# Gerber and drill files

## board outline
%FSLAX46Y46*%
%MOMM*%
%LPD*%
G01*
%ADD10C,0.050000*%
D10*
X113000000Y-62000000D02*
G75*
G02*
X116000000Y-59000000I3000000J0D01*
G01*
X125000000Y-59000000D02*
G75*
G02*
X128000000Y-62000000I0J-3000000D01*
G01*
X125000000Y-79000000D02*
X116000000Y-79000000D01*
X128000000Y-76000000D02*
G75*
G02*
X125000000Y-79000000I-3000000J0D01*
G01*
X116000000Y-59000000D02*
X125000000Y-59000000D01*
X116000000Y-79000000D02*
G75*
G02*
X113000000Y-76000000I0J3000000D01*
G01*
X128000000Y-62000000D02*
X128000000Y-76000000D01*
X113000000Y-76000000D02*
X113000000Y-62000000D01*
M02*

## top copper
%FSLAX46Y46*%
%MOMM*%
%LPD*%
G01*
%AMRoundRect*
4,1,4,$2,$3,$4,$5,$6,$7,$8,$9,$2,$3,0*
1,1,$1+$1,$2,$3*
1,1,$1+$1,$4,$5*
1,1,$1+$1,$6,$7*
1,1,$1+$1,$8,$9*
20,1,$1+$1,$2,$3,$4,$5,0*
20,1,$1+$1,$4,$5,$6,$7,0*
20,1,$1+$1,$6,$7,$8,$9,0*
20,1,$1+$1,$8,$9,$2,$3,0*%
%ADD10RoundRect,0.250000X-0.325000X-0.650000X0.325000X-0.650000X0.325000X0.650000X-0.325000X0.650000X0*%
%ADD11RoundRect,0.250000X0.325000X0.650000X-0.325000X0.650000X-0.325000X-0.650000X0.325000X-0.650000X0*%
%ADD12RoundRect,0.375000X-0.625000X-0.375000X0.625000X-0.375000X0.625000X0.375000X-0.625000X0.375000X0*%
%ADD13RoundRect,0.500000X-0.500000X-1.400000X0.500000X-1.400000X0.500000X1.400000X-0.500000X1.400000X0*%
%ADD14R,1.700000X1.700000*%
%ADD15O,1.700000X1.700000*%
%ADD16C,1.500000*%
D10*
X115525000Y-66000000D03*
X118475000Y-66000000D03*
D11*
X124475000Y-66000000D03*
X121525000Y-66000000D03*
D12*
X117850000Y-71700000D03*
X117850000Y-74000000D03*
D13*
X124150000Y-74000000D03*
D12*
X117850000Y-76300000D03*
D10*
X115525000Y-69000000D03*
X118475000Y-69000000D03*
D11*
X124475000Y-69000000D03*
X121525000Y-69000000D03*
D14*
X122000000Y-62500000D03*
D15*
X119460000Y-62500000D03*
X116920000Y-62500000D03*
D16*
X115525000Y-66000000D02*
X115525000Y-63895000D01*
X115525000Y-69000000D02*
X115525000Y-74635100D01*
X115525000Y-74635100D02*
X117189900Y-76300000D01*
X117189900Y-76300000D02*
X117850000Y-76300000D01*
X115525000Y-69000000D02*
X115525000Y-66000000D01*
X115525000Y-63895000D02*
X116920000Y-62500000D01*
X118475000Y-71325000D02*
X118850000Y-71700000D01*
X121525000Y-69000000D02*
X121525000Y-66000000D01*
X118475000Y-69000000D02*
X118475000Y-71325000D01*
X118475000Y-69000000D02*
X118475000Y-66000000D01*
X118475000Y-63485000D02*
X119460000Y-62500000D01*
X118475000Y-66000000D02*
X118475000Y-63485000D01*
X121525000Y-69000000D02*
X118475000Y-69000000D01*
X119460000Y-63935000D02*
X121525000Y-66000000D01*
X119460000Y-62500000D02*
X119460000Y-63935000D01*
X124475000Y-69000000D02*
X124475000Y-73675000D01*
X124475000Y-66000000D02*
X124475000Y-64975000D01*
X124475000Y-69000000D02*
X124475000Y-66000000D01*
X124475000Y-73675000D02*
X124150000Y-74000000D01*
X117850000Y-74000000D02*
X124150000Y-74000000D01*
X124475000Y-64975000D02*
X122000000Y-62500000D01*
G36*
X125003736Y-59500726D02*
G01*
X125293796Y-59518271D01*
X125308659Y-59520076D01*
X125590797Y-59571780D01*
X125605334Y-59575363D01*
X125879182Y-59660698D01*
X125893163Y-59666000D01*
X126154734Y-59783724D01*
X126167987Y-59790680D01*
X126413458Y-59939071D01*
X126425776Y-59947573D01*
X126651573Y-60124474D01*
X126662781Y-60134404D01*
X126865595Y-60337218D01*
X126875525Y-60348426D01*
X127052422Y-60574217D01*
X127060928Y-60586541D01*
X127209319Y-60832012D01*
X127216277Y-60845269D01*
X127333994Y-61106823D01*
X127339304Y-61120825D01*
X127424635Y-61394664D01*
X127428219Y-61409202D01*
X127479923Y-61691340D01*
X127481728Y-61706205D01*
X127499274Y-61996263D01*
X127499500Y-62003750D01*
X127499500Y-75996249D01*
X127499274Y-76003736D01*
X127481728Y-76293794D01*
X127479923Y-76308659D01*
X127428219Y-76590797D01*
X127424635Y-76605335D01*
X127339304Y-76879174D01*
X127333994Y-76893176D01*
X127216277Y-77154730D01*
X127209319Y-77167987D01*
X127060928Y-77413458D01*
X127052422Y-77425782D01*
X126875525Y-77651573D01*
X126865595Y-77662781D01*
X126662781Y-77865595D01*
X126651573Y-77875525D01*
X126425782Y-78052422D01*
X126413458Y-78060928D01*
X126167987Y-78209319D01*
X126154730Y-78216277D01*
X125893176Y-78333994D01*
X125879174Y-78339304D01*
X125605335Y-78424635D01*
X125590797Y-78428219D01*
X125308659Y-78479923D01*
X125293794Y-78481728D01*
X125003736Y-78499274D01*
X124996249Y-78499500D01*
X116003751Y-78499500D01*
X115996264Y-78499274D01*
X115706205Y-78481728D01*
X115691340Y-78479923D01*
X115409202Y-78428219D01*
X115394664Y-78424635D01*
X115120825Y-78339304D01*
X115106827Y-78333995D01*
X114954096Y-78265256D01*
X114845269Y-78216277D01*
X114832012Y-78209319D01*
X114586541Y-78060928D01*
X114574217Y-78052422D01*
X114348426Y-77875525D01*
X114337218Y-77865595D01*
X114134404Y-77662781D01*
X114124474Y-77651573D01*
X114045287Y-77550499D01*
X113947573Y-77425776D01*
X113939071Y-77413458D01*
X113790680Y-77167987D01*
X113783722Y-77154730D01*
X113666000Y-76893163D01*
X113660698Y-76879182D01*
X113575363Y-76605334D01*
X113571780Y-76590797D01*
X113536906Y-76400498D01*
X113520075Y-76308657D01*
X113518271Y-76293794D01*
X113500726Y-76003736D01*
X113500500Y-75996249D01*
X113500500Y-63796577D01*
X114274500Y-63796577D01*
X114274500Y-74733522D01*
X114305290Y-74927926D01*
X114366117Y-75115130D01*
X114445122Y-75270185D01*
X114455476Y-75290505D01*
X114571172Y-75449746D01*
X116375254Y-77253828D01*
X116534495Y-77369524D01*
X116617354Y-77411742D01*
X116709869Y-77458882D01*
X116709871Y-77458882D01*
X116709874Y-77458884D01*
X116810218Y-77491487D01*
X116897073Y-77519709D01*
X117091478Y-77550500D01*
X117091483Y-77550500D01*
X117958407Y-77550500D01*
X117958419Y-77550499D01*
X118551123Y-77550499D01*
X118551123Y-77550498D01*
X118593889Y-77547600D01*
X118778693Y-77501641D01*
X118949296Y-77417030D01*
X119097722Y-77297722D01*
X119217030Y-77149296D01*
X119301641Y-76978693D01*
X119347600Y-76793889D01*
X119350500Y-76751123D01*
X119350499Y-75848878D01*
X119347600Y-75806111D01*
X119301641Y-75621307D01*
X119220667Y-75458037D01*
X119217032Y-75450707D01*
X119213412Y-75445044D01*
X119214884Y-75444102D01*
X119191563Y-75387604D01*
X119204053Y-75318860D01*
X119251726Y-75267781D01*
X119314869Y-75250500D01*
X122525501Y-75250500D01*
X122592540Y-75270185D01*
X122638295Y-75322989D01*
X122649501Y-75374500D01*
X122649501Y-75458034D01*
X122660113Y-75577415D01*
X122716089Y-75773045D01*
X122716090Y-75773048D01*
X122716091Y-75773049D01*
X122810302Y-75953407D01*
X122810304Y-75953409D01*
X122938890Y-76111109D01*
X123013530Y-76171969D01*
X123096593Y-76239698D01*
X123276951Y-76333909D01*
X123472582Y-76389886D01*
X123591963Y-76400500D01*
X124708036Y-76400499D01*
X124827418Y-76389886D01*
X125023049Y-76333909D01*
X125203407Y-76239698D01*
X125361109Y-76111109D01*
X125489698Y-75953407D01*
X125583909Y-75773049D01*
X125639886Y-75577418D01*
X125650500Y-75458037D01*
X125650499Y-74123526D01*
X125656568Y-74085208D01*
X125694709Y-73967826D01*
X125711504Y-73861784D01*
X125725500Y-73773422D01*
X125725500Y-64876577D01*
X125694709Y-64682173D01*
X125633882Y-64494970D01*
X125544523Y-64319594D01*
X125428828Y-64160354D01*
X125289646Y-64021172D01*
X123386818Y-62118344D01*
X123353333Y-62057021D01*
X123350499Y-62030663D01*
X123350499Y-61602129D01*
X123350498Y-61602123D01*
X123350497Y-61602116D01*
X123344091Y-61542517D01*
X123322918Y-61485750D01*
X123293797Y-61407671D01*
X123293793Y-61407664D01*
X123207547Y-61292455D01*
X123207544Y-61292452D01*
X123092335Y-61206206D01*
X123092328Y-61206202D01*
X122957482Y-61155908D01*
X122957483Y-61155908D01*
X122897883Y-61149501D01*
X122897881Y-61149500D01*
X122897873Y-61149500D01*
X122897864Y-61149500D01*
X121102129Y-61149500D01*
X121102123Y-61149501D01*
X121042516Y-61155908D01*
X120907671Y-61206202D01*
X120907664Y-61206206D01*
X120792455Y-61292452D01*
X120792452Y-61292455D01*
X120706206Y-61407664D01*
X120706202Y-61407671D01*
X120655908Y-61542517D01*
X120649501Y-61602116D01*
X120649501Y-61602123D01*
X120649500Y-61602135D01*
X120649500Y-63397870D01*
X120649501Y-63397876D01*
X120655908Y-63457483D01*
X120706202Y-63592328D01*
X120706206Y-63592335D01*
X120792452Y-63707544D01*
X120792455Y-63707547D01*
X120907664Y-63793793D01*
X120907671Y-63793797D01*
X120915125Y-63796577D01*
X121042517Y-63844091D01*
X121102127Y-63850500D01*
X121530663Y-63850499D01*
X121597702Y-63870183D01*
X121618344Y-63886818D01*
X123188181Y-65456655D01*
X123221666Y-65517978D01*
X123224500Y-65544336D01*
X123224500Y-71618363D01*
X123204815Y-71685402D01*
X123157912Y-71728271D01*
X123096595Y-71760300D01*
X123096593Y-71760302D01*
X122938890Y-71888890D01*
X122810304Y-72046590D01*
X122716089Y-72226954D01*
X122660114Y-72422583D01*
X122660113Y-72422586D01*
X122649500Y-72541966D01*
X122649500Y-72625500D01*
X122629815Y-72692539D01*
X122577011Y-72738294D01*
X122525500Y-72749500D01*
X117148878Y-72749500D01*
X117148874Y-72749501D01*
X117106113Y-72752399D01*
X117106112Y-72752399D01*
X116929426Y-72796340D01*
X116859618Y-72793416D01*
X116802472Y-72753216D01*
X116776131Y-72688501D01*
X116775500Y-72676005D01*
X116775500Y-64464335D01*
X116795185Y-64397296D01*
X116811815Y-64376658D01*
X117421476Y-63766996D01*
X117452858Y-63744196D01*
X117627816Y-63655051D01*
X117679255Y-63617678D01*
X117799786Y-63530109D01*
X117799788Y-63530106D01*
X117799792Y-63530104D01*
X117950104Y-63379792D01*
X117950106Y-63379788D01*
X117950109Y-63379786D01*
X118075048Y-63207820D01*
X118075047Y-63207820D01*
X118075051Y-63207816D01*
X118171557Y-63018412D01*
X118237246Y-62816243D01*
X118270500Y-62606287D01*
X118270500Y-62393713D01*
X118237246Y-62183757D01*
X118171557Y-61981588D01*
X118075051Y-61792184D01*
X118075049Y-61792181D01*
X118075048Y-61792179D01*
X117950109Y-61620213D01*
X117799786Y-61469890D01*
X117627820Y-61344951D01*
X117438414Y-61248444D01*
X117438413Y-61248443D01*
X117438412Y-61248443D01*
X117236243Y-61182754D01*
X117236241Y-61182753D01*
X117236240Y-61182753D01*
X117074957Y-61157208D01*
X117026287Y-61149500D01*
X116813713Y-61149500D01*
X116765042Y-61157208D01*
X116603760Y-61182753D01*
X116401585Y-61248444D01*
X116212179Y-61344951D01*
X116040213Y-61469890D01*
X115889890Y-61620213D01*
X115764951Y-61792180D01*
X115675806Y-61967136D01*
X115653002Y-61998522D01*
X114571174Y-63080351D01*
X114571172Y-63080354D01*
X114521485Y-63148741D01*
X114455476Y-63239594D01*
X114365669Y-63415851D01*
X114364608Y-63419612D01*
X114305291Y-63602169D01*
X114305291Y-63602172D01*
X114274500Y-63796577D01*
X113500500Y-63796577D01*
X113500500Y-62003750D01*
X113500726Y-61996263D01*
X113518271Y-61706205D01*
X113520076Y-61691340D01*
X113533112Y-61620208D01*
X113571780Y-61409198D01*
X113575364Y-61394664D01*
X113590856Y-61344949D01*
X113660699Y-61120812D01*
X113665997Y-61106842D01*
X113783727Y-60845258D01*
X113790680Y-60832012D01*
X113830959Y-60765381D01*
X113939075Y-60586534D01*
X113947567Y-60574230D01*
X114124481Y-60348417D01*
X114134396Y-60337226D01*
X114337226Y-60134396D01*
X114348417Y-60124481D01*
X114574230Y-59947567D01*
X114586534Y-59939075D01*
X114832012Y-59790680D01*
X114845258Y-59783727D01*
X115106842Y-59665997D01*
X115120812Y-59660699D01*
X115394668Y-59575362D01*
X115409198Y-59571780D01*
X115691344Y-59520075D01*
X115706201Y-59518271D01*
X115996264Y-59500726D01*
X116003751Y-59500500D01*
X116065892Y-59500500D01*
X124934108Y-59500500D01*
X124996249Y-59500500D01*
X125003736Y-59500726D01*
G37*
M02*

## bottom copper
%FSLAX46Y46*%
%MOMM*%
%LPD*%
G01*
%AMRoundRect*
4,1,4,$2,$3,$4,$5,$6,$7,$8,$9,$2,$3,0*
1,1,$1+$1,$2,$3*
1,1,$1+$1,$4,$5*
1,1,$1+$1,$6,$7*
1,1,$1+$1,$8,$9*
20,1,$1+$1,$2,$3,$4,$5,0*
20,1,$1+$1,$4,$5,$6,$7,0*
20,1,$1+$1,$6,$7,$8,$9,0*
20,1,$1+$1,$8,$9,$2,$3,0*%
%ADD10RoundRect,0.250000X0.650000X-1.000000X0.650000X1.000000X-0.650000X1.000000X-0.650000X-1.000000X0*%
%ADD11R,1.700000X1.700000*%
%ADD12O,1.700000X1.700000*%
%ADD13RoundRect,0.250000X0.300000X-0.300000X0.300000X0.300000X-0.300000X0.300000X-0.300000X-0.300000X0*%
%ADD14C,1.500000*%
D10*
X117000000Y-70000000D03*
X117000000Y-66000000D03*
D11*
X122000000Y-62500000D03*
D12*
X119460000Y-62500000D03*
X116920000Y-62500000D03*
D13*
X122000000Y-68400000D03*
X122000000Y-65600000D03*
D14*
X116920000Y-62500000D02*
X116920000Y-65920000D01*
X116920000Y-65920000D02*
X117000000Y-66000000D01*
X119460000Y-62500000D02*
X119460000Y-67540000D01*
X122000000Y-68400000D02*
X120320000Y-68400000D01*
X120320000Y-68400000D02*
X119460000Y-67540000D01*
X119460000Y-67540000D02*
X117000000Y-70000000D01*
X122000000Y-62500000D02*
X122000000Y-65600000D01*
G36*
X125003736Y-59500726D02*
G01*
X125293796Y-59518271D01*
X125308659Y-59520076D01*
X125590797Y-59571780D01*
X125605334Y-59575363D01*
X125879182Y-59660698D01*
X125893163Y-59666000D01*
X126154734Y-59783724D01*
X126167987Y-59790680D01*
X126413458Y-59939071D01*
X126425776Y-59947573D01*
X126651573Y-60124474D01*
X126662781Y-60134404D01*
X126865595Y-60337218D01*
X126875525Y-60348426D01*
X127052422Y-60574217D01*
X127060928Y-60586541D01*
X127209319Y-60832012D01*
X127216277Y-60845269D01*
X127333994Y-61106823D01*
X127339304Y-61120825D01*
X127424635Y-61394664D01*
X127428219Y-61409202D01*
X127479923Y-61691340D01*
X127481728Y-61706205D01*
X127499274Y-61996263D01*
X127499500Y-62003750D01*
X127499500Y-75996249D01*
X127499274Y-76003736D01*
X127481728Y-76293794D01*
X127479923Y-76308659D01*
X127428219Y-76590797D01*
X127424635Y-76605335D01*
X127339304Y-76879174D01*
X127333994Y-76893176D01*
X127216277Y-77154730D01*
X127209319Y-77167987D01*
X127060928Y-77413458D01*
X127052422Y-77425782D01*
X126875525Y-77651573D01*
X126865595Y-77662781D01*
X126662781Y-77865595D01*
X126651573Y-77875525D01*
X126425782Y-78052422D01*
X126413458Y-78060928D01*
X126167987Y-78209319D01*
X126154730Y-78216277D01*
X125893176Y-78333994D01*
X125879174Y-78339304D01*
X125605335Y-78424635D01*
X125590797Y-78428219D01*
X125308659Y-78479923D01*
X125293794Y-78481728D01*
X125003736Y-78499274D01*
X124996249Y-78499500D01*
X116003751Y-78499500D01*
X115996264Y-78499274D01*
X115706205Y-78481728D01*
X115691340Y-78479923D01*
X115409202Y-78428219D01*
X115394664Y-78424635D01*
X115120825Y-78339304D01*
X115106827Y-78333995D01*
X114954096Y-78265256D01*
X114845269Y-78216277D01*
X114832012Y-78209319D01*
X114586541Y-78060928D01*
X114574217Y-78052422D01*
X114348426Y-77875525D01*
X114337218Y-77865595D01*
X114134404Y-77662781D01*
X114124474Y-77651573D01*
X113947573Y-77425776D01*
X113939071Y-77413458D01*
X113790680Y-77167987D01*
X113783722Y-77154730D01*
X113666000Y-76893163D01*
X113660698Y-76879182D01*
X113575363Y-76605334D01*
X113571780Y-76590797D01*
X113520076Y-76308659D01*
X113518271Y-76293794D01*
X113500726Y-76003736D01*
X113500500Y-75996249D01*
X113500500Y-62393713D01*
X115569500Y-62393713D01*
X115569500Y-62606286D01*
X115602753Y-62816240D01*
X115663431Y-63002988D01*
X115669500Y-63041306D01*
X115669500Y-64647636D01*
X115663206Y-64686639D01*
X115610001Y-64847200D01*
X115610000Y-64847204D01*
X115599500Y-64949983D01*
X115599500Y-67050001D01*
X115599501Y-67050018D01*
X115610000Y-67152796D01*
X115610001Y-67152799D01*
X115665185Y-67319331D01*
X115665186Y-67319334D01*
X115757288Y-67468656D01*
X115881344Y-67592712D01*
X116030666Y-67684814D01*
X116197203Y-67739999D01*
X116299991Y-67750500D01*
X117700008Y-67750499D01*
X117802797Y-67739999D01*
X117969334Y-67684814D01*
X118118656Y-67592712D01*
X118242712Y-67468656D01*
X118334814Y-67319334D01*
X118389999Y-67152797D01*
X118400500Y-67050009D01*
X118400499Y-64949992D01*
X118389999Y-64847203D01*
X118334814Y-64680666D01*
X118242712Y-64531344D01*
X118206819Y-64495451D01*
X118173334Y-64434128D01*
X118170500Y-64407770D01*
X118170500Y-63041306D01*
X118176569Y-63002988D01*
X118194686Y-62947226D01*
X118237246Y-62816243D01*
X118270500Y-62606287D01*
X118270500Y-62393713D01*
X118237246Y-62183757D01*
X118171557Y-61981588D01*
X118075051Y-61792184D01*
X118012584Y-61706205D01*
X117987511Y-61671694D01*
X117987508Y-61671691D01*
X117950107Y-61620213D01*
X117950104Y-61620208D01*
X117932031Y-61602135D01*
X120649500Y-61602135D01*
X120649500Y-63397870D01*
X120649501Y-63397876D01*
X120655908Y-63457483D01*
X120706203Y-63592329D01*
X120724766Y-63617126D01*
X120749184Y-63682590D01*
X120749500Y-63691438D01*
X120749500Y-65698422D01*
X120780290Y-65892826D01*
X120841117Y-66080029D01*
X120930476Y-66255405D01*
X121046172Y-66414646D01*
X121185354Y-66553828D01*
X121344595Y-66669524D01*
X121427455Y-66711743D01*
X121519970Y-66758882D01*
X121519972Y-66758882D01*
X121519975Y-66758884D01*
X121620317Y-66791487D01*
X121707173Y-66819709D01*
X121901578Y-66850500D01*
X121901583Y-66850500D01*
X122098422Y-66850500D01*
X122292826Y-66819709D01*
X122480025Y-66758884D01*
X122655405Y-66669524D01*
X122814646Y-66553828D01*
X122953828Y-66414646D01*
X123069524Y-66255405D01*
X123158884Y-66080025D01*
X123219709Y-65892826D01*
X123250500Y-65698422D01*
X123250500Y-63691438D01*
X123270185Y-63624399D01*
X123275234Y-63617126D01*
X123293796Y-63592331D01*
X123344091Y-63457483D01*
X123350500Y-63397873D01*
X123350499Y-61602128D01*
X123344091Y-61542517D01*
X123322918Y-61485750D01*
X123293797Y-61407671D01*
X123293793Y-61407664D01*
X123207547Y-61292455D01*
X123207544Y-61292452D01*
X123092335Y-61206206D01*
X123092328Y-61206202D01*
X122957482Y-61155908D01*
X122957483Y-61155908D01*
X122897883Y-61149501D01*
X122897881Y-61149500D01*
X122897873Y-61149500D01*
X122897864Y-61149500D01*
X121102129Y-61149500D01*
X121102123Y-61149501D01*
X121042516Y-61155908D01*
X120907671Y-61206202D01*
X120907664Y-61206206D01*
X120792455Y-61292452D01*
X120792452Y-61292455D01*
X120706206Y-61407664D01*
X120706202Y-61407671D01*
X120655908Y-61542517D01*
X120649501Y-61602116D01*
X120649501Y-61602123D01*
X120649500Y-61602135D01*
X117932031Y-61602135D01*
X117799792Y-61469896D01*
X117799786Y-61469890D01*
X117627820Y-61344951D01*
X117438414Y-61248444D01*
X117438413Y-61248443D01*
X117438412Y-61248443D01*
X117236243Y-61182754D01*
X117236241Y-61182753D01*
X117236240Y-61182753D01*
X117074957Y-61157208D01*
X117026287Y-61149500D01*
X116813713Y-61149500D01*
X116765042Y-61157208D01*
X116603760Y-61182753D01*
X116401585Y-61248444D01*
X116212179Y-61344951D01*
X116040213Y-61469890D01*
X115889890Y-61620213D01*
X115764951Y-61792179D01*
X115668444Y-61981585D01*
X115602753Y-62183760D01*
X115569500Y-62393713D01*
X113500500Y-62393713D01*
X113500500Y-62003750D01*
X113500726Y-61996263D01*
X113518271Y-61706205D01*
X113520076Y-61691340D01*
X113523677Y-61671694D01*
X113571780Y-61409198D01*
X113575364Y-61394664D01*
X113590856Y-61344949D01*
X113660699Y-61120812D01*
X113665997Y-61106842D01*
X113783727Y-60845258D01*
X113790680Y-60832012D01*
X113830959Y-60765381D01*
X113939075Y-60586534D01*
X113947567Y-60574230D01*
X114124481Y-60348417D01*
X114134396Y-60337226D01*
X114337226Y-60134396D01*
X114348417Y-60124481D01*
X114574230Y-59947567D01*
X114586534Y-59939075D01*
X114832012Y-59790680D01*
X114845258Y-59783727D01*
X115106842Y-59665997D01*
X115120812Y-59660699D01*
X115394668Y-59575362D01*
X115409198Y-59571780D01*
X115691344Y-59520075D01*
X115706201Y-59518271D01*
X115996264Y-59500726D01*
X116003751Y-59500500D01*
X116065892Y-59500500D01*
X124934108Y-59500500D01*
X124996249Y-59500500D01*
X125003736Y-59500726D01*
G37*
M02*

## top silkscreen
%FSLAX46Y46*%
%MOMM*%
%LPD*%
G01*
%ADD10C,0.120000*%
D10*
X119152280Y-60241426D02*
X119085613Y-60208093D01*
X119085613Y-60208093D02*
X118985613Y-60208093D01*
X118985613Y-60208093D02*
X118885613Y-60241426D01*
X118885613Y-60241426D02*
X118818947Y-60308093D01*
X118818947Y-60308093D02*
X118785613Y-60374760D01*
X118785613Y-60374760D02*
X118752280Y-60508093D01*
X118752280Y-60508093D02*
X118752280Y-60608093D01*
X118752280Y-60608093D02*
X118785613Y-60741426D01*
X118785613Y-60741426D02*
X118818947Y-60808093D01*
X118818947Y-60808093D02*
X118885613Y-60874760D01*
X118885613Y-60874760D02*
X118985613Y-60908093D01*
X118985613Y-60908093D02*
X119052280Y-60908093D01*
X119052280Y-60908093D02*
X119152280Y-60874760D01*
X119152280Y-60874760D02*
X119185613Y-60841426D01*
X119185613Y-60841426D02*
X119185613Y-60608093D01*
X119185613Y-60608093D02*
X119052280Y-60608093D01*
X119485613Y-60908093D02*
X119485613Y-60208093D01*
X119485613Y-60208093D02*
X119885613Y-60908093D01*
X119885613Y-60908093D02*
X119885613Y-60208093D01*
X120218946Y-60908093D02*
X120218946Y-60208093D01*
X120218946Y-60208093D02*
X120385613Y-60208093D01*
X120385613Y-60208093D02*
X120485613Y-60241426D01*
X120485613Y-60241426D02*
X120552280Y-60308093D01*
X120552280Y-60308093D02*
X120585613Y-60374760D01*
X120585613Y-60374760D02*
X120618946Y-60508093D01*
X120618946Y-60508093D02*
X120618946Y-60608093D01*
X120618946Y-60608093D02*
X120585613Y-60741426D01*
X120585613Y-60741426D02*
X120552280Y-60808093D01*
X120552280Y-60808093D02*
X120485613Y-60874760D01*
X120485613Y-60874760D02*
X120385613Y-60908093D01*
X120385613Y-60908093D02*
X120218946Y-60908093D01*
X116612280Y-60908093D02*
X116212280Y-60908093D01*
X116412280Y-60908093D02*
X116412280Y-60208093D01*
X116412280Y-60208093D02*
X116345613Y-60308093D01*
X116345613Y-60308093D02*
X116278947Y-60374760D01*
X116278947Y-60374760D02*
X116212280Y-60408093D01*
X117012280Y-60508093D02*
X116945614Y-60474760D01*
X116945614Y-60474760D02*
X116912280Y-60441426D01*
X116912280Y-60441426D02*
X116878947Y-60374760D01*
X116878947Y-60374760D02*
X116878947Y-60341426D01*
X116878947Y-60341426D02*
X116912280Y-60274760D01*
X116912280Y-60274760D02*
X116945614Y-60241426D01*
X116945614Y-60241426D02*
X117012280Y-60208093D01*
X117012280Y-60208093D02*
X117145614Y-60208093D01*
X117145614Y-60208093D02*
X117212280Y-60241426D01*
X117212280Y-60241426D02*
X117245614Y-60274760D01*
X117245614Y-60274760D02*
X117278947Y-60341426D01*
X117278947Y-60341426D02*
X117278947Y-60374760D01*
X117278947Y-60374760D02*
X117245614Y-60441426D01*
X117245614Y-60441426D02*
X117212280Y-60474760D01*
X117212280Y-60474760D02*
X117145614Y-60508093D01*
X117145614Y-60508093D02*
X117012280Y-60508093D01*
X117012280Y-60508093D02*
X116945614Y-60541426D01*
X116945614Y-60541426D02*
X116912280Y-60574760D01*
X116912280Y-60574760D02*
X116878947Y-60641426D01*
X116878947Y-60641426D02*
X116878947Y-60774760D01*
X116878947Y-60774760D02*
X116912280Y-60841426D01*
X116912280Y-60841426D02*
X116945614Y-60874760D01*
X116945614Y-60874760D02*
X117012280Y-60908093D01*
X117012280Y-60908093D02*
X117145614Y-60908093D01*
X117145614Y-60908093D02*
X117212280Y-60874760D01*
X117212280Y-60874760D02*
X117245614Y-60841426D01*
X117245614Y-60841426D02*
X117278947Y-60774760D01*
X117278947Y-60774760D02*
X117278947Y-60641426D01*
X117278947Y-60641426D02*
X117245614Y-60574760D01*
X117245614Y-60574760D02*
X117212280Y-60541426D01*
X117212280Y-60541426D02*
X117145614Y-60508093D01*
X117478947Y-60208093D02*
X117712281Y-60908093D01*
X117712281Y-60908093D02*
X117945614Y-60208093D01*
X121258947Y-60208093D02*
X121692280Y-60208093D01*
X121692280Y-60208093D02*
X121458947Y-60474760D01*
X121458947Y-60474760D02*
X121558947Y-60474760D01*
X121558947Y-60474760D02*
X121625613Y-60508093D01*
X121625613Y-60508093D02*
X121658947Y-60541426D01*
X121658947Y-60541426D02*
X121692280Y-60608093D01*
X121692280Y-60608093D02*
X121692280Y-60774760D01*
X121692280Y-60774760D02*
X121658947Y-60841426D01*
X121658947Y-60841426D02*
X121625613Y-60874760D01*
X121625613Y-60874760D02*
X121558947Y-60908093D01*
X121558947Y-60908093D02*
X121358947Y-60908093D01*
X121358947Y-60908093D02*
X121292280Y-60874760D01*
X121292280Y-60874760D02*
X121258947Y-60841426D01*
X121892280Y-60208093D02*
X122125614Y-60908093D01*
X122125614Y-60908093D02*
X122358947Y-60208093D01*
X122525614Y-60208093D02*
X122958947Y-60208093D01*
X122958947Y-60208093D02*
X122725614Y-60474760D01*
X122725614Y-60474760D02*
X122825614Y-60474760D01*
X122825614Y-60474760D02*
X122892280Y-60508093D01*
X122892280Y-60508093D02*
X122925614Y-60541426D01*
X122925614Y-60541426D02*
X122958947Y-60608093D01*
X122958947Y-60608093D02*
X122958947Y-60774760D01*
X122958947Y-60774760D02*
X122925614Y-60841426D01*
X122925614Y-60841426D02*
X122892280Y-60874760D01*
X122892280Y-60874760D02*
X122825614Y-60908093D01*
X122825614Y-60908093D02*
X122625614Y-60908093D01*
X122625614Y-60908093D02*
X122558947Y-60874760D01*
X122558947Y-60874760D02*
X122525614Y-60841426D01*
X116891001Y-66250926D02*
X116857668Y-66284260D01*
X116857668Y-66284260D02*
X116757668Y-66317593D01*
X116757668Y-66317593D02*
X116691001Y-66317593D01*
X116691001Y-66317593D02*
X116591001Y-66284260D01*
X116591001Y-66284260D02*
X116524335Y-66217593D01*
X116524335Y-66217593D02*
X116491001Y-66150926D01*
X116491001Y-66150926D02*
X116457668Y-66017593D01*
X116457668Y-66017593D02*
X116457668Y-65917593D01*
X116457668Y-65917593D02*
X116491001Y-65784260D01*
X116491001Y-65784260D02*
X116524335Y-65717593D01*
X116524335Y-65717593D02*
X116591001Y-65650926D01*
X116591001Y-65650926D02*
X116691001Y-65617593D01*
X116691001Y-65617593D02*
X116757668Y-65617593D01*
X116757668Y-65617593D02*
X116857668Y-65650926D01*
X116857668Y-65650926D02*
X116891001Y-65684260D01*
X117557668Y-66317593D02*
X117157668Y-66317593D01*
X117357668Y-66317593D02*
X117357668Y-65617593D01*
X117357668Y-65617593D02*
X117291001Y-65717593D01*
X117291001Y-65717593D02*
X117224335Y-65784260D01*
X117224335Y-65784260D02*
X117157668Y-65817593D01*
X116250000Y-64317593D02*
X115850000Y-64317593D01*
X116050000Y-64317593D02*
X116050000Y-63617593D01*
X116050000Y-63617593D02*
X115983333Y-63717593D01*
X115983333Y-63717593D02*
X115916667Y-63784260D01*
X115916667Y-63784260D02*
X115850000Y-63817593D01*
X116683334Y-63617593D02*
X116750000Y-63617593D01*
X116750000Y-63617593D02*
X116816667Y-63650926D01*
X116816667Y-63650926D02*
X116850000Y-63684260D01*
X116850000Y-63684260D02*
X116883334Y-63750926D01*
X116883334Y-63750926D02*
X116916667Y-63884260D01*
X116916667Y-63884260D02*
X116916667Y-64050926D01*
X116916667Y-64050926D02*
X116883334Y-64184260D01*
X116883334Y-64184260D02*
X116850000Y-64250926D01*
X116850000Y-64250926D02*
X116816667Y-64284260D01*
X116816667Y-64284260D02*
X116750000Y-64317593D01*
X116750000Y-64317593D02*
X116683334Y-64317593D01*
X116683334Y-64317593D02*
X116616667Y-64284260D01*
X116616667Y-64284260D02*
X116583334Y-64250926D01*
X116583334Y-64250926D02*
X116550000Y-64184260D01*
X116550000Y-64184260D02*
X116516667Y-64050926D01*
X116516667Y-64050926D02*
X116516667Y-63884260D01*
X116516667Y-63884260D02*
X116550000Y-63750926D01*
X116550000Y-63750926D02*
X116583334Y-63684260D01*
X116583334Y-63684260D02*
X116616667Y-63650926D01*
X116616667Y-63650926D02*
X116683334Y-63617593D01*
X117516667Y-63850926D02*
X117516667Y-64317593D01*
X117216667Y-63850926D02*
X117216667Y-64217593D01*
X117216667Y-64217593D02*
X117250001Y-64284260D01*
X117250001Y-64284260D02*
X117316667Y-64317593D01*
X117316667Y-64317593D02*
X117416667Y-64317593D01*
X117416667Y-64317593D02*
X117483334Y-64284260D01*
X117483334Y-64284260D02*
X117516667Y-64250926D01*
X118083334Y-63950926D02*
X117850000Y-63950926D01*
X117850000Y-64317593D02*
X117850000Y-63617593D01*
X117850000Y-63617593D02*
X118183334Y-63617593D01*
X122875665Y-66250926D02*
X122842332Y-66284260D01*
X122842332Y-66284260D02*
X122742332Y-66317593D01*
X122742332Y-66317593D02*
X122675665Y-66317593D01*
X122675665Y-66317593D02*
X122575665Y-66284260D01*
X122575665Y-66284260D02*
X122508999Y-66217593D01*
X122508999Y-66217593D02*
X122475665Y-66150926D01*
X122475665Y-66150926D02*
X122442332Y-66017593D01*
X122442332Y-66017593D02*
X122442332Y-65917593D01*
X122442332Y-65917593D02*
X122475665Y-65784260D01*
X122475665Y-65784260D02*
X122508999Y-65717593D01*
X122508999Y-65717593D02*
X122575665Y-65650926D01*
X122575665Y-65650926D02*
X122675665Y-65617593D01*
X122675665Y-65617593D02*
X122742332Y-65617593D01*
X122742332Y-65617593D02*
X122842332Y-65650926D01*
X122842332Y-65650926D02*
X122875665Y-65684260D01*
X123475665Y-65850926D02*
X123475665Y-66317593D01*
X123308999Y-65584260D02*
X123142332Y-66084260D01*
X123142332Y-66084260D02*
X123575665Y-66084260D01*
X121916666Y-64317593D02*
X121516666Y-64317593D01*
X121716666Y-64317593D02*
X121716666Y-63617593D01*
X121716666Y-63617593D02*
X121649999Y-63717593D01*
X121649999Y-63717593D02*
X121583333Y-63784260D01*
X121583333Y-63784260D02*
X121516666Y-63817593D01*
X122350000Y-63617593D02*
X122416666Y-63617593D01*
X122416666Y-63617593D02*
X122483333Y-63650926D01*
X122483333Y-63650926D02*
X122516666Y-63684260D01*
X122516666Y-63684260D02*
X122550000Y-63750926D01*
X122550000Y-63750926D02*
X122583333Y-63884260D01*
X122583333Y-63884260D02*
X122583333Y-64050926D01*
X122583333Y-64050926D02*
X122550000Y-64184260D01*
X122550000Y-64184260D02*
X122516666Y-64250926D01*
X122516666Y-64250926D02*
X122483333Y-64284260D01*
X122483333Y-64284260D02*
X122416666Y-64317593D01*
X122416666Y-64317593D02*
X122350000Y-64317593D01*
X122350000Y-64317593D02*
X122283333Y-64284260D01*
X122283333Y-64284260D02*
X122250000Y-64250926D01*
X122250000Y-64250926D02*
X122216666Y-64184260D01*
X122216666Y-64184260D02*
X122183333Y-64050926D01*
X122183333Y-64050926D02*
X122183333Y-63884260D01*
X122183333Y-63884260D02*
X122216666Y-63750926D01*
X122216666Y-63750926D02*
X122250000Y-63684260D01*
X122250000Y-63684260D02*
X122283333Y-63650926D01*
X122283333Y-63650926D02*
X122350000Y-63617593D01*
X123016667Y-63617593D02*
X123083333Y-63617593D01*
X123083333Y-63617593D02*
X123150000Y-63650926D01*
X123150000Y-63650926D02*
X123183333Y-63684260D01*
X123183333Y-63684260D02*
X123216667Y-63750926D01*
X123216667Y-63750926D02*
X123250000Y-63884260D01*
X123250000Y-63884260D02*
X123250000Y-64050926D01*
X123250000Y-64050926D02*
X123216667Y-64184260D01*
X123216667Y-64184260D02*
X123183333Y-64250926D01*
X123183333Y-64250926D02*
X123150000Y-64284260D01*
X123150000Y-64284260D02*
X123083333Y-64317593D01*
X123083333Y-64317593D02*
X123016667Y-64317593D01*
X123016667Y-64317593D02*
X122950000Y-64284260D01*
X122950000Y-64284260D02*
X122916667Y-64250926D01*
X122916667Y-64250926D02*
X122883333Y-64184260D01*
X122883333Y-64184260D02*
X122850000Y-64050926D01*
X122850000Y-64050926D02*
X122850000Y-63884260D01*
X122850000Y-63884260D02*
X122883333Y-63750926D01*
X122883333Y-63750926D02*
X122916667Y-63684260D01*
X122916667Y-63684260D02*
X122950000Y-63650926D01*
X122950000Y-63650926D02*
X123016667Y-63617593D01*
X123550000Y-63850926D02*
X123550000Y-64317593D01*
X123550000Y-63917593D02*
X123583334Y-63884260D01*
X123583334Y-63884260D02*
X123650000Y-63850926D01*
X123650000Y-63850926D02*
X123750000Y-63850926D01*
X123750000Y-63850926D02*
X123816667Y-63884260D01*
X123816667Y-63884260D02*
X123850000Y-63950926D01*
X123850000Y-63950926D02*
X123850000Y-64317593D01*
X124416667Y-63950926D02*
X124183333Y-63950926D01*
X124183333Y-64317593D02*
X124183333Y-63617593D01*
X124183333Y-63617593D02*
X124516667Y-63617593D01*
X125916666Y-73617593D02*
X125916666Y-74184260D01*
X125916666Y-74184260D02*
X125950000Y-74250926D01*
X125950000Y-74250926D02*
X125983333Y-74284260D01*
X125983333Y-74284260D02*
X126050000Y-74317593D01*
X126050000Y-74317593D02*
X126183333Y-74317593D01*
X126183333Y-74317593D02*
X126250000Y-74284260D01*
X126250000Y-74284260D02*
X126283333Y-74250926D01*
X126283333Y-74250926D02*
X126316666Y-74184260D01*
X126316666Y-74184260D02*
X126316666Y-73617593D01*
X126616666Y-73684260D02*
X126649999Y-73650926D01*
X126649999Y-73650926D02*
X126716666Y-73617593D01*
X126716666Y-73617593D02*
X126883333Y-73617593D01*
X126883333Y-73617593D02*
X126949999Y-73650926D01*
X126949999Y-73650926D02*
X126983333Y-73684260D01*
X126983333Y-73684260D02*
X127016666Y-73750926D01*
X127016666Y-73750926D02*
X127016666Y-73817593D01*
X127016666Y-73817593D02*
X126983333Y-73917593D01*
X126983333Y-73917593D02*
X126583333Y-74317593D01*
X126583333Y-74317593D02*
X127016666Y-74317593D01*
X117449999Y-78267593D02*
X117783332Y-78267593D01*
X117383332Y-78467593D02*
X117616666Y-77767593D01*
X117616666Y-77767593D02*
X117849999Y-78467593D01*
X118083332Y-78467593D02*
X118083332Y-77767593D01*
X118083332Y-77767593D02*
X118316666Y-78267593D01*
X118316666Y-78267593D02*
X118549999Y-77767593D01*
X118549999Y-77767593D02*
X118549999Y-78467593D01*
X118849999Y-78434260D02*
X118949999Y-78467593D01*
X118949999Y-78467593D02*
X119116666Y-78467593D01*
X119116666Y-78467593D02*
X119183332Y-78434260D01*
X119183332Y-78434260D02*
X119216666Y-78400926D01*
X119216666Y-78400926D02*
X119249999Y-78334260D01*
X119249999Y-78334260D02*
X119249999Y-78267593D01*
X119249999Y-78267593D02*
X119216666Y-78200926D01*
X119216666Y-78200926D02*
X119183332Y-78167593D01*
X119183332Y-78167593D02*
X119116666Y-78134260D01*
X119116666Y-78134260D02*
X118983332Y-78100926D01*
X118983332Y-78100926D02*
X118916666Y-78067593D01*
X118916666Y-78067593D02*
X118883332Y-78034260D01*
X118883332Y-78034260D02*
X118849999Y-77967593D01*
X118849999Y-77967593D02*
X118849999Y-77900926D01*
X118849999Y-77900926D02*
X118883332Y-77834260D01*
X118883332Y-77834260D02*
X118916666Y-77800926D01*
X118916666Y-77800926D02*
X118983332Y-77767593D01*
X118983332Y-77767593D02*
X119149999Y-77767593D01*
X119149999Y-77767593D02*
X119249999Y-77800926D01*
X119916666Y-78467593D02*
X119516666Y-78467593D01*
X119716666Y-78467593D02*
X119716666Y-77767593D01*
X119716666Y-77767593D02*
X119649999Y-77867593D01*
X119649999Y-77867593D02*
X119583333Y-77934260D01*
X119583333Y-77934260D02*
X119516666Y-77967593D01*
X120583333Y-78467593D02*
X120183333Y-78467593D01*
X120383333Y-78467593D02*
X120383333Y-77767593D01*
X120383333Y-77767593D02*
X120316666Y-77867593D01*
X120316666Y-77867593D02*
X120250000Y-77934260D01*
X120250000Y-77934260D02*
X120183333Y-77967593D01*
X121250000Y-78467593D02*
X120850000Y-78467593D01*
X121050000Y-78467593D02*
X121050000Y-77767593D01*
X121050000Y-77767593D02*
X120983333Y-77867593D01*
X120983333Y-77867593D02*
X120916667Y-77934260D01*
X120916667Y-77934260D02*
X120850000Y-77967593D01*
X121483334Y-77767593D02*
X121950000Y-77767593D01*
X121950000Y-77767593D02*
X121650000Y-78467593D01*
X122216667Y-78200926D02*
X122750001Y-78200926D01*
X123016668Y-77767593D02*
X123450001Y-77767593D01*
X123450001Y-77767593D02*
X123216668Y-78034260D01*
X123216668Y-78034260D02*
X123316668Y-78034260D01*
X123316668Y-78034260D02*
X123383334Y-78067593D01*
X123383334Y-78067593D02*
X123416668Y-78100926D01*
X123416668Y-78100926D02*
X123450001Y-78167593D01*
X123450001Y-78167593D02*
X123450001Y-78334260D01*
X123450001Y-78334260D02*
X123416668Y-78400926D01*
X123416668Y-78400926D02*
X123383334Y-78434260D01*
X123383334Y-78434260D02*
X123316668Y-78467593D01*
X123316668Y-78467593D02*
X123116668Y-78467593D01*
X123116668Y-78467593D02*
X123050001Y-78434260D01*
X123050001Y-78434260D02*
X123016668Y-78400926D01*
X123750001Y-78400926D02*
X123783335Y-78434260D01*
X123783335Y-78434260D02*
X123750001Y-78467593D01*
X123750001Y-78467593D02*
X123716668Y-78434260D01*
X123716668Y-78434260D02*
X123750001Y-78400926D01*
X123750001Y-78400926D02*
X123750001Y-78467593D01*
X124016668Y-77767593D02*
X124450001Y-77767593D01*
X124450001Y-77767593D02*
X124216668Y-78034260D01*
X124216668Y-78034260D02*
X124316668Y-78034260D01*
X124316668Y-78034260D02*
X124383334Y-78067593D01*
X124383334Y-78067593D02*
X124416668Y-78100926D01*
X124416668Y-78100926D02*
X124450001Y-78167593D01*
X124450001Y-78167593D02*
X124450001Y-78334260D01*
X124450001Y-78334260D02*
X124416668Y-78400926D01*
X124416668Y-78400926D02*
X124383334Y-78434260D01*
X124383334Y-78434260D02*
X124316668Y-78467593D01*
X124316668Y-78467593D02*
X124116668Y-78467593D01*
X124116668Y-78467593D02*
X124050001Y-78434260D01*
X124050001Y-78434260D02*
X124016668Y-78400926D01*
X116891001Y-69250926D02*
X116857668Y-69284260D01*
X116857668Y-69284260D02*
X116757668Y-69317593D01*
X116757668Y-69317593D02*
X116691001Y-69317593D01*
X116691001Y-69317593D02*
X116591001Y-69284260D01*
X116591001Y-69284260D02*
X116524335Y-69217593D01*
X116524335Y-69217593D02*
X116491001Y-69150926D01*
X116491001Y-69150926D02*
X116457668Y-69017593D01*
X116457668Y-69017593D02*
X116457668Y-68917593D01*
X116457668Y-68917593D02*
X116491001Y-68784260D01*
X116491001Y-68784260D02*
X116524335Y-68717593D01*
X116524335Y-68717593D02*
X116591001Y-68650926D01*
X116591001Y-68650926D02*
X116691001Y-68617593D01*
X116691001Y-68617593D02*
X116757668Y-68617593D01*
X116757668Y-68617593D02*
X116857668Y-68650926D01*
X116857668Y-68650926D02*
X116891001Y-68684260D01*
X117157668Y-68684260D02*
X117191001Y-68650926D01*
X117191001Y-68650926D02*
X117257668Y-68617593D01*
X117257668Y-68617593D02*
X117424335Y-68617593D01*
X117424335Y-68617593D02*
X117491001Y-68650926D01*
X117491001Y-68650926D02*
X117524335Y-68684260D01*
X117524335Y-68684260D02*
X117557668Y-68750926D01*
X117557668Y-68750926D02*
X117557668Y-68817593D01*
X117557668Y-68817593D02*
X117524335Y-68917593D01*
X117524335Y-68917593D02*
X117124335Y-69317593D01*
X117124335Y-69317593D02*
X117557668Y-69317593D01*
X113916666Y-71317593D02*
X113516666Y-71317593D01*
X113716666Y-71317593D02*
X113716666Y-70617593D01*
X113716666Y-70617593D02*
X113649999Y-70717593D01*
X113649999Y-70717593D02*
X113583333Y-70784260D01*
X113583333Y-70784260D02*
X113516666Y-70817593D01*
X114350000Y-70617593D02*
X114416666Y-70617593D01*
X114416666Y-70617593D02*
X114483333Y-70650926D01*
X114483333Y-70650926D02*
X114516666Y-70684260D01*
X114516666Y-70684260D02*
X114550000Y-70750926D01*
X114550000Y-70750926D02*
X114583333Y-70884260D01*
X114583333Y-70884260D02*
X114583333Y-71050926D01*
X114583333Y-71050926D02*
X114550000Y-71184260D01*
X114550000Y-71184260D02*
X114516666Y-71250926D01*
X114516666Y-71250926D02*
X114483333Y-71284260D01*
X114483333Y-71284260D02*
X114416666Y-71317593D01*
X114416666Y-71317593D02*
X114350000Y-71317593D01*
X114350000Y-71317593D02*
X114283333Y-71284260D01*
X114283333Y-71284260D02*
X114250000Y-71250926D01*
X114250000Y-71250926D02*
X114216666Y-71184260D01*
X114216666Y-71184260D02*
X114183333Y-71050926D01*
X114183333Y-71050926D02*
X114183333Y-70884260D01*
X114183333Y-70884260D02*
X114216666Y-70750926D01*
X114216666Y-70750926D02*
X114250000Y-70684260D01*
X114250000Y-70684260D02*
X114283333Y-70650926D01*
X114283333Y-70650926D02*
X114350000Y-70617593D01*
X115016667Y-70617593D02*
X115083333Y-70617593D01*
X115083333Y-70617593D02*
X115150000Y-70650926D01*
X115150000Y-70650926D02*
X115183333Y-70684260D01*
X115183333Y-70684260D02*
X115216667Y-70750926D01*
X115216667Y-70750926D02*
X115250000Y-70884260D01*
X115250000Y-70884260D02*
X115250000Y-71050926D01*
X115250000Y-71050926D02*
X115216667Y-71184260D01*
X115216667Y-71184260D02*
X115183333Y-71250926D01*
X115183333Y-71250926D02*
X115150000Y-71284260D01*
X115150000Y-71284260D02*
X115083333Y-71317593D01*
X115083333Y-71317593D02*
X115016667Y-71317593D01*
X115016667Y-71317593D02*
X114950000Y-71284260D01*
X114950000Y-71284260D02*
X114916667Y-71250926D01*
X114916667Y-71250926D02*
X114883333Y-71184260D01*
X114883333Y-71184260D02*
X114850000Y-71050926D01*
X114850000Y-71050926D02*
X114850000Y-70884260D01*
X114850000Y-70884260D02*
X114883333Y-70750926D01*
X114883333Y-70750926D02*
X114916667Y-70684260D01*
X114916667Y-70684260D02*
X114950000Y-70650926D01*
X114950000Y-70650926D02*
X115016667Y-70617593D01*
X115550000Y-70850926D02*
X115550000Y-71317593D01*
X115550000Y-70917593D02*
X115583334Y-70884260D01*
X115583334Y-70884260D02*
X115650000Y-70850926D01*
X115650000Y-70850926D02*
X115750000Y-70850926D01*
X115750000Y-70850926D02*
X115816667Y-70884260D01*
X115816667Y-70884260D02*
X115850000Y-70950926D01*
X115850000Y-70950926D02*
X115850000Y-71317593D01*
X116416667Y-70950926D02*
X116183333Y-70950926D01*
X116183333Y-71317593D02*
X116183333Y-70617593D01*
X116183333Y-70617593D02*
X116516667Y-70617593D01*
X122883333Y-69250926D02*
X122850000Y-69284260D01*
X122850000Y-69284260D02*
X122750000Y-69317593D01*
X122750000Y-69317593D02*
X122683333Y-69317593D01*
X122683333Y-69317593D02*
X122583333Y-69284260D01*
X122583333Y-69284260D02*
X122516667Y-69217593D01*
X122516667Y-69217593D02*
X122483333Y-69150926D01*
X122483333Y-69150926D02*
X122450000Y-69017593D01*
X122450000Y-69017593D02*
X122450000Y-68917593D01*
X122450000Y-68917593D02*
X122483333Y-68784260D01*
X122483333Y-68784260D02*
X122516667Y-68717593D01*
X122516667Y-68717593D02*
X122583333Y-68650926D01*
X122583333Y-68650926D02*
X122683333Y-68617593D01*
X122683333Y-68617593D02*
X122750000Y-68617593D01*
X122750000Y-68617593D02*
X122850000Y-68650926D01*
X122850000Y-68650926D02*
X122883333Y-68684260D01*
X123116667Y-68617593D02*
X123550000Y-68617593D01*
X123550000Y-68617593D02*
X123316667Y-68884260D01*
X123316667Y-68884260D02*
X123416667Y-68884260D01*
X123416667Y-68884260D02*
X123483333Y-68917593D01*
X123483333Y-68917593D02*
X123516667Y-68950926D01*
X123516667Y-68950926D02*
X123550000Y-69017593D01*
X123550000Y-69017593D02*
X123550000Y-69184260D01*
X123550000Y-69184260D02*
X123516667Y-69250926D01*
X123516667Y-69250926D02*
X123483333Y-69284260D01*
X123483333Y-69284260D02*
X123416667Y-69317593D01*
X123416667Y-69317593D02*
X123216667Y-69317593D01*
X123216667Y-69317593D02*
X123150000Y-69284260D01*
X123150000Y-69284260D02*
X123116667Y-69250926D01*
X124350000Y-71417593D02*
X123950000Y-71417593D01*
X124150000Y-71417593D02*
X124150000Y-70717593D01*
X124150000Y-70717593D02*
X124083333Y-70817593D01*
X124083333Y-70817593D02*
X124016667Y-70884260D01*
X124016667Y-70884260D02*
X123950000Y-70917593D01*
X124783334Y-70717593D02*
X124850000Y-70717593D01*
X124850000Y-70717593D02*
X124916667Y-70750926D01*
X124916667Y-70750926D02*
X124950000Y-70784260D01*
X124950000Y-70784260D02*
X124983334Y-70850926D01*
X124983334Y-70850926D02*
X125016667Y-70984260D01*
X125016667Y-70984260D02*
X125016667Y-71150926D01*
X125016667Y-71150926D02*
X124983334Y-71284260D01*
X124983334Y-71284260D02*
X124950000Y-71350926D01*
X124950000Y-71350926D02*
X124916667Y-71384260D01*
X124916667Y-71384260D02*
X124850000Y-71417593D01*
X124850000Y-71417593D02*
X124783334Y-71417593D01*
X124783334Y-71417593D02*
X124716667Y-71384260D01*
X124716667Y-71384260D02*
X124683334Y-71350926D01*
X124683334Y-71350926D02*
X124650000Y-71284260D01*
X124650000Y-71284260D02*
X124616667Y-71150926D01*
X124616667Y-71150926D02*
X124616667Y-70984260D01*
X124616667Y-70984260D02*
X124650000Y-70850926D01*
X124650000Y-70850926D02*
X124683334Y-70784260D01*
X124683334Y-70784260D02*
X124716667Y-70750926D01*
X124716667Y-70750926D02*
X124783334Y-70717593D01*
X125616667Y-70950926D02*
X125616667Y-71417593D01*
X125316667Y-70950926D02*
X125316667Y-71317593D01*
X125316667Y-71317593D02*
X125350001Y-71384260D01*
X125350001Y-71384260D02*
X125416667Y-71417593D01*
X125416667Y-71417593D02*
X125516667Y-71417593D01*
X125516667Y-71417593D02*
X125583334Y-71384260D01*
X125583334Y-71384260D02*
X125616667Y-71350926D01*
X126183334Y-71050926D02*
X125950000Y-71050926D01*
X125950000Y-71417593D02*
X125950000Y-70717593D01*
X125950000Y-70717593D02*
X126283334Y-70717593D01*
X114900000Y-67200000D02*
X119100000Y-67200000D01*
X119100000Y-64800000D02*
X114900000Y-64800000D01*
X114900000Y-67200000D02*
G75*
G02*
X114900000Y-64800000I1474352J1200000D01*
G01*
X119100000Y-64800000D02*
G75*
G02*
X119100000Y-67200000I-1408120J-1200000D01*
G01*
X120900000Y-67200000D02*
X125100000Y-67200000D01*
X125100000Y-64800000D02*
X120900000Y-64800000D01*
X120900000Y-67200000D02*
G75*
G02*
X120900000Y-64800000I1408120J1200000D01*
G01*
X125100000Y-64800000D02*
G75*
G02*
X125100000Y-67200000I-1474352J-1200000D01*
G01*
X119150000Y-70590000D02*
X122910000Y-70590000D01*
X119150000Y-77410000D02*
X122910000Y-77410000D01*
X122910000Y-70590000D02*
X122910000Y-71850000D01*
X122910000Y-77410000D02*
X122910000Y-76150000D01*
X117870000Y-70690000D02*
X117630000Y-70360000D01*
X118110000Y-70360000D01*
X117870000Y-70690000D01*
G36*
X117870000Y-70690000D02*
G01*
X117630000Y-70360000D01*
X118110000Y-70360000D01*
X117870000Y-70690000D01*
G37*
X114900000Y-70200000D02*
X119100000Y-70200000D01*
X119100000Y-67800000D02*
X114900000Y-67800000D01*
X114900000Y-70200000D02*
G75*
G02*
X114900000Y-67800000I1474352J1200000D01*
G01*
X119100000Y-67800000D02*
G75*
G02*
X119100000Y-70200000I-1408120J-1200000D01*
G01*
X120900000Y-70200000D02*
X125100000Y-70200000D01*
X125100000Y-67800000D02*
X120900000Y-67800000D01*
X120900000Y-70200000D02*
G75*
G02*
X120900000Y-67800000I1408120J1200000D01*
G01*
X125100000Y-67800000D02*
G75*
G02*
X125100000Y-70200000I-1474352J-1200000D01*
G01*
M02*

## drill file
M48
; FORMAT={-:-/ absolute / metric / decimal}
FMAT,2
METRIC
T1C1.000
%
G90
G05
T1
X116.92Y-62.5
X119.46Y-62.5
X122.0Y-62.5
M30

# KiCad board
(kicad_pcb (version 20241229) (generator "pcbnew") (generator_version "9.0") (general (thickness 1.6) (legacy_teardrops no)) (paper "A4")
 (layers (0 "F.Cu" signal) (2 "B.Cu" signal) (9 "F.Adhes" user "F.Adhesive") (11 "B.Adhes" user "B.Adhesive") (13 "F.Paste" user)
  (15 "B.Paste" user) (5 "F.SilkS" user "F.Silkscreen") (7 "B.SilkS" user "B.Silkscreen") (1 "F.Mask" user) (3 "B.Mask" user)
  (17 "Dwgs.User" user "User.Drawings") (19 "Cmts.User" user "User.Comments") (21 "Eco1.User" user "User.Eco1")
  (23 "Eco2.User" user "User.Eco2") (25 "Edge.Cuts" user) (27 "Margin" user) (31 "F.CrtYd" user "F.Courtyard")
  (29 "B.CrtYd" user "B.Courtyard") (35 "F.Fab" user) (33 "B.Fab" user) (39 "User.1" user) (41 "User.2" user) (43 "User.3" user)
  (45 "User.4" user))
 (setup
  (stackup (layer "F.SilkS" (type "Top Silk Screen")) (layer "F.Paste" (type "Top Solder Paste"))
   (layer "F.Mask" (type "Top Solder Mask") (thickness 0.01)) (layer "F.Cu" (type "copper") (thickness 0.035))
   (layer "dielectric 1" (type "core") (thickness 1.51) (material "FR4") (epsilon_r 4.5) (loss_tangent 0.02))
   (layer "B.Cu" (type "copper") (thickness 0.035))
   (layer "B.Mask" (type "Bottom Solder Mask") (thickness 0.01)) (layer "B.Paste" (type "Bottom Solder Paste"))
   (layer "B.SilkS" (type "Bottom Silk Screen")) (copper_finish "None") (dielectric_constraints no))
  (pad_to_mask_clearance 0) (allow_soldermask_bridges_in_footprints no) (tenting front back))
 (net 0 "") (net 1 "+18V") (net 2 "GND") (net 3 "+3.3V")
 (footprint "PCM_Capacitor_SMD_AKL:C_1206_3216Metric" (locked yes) (layer "F.Cu") (at 117 66)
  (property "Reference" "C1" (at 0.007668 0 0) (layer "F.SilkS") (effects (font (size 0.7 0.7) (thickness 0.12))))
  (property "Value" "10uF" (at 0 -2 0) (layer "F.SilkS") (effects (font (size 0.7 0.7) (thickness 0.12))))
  (fp_line (start -2.1 1.2) (end 2.1 1.2) (stroke (width 0.12) (type solid)) (layer "F.SilkS"))
  (fp_line (start 2.1 -1.2) (end -2.1 -1.2) (stroke (width 0.12) (type solid)) (layer "F.SilkS"))
  (fp_arc (start -2.1 1.2) (mid -2.526625 0) (end -2.1 -1.2) (stroke (width 0.12) (type solid)) (layer "F.SilkS"))
  (fp_arc (start 2.1 -1.2) (mid 2.541962 0) (end 2.1 1.2) (stroke (width 0.12) (type solid)) (layer "F.SilkS"))
  (pad "1" smd roundrect (at -1.475 0) (size 1.15 1.8) (layers "F.Cu" "F.Mask" "F.Paste") (roundrect_rratio 0.217391) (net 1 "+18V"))
  (pad "2" smd roundrect (at 1.475 0) (size 1.15 1.8) (layers "F.Cu" "F.Mask" "F.Paste") (roundrect_rratio 0.217391) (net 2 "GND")))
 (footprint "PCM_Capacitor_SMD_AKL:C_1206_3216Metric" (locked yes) (layer "F.Cu") (at 123 66 180)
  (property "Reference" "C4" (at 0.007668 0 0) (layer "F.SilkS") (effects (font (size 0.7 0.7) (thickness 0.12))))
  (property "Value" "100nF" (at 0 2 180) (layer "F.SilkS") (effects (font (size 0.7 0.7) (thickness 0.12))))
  (fp_line (start 2.1 -1.2) (end -2.1 -1.2) (stroke (width 0.12) (type solid)) (layer "F.SilkS"))
  (fp_line (start -2.1 1.2) (end 2.1 1.2) (stroke (width 0.12) (type solid)) (layer "F.SilkS"))
  (fp_arc (start 2.1 -1.2) (mid 2.541962 0) (end 2.1 1.2) (stroke (width 0.12) (type solid)) (layer "F.SilkS"))
  (fp_arc (start -2.1 1.2) (mid -2.526625 0) (end -2.1 -1.2) (stroke (width 0.12) (type solid)) (layer "F.SilkS"))
  (pad "1" smd roundrect (at -1.475 0 180) (size 1.15 1.8) (layers "F.Cu" "F.Mask" "F.Paste") (roundrect_rratio 0.217391) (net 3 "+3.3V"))
  (pad "2" smd roundrect (at 1.475 0 180) (size 1.15 1.8) (layers "F.Cu" "F.Mask" "F.Paste") (roundrect_rratio 0.217391) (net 2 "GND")))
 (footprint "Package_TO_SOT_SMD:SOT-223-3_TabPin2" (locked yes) (layer "F.Cu") (at 121 74)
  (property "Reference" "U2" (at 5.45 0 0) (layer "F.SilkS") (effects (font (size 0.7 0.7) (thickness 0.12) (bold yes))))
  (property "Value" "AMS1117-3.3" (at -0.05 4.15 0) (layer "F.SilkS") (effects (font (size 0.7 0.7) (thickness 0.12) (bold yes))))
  (fp_line (start -1.85 -3.41) (end 1.91 -3.41) (stroke (width 0.12) (type solid)) (layer "F.SilkS"))
  (fp_line (start -1.85 3.41) (end 1.91 3.41) (stroke (width 0.12) (type solid)) (layer "F.SilkS"))
  (fp_line (start 1.91 -3.41) (end 1.91 -2.15) (stroke (width 0.12) (type solid)) (layer "F.SilkS"))
  (fp_line (start 1.91 3.41) (end 1.91 2.15) (stroke (width 0.12) (type solid)) (layer "F.SilkS"))
  (fp_poly
   (pts (xy -3.13 -3.31) (xy -3.37 -3.64) (xy -2.89 -3.64) (xy -3.13 -3.31)) (stroke (width 0.12) (type solid)) (fill yes) (layer "F.SilkS"))
  (pad "1" smd roundrect (at -3.15 -2.3) (size 2 1.5) (layers "F.Cu" "F.Mask" "F.Paste") (roundrect_rratio 0.25) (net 2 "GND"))
  (pad "2" smd roundrect (at -3.15 0) (size 2 1.5) (layers "F.Cu" "F.Mask" "F.Paste") (roundrect_rratio 0.25) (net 3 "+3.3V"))
  (pad "2" smd roundrect (at 3.15 0) (size 2 3.8) (layers "F.Cu" "F.Mask" "F.Paste") (roundrect_rratio 0.25) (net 3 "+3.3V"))
  (pad "3" smd roundrect (at -3.15 2.3) (size 2 1.5) (layers "F.Cu" "F.Mask" "F.Paste") (roundrect_rratio 0.25) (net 1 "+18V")))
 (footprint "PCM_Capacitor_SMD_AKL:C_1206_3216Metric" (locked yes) (layer "F.Cu") (at 117 69)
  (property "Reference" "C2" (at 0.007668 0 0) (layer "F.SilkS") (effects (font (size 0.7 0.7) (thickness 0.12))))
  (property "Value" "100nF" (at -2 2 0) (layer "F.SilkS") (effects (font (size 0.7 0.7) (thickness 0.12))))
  (fp_line (start -2.1 1.2) (end 2.1 1.2) (stroke (width 0.12) (type solid)) (layer "F.SilkS"))
  (fp_line (start 2.1 -1.2) (end -2.1 -1.2) (stroke (width 0.12) (type solid)) (layer "F.SilkS"))
  (fp_arc (start -2.1 1.2) (mid -2.526625 0) (end -2.1 -1.2) (stroke (width 0.12) (type solid)) (layer "F.SilkS"))
  (fp_arc (start 2.1 -1.2) (mid 2.541962 0) (end 2.1 1.2) (stroke (width 0.12) (type solid)) (layer "F.SilkS"))
  (pad "1" smd roundrect (at -1.475 0) (size 1.15 1.8) (layers "F.Cu" "F.Mask" "F.Paste") (roundrect_rratio 0.217391) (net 1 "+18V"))
  (pad "2" smd roundrect (at 1.475 0) (size 1.15 1.8) (layers "F.Cu" "F.Mask" "F.Paste") (roundrect_rratio 0.217391) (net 2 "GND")))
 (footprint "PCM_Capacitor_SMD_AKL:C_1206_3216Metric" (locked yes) (layer "F.Cu") (at 123 69 180)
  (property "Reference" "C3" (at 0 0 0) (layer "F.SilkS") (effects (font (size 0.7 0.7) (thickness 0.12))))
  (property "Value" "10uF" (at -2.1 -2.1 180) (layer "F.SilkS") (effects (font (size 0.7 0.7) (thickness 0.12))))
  (fp_line (start 2.1 -1.2) (end -2.1 -1.2) (stroke (width 0.12) (type solid)) (layer "F.SilkS"))
  (fp_line (start -2.1 1.2) (end 2.1 1.2) (stroke (width 0.12) (type solid)) (layer "F.SilkS"))
  (fp_arc (start 2.1 -1.2) (mid 2.541962 0) (end 2.1 1.2) (stroke (width 0.12) (type solid)) (layer "F.SilkS"))
  (fp_arc (start -2.1 1.2) (mid -2.526625 0) (end -2.1 -1.2) (stroke (width 0.12) (type solid)) (layer "F.SilkS"))
  (pad "1" smd roundrect (at -1.475 0 180) (size 1.15 1.8) (layers "F.Cu" "F.Mask" "F.Paste") (roundrect_rratio 0.217391) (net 3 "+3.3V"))
  (pad "2" smd roundrect (at 1.475 0 180) (size 1.15 1.8) (layers "F.Cu" "F.Mask" "F.Paste") (roundrect_rratio 0.217391) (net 2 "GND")))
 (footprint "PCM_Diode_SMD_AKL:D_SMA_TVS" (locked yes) (layer "B.Cu") (at 117 68 90)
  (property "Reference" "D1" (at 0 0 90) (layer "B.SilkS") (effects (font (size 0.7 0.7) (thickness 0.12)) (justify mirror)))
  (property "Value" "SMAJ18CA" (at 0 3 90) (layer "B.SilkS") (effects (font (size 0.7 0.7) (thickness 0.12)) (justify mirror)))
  (pad "1" smd roundrect (at -2 0 90) (size 2.5 1.8) (layers "B.Cu" "B.Mask" "B.Paste") (roundrect_rratio 0.1388888889) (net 2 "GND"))
  (pad "2" smd roundrect (at 2 0 90) (size 2.5 1.8) (layers "B.Cu" "B.Mask" "B.Paste") (roundrect_rratio 0.1388888889) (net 1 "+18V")))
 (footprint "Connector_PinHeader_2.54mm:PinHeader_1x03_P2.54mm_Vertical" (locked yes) (layer "B.Cu") (at 122 62.5 90)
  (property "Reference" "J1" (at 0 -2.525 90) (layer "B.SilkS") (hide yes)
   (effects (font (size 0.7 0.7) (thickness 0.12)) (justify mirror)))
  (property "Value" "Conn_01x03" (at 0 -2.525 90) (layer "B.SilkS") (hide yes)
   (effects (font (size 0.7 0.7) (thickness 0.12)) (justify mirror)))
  (pad "1" thru_hole rect (at 0 0 90) (size 1.7 1.7) (drill 1) (layers "*.Cu" "*.Mask") (remove_unused_layers no) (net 3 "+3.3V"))
  (pad "2" thru_hole oval (at 0 -2.54 90) (size 1.7 1.7) (drill 1) (layers "*.Cu" "*.Mask") (remove_unused_layers no) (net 2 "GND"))
  (pad "3" thru_hole oval (at 0 -5.08 90) (size 1.7 1.7) (drill 1) (layers "*.Cu" "*.Mask") (remove_unused_layers no) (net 1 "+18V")))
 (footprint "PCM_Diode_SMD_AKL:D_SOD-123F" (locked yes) (layer "B.Cu") (at 122 67 90)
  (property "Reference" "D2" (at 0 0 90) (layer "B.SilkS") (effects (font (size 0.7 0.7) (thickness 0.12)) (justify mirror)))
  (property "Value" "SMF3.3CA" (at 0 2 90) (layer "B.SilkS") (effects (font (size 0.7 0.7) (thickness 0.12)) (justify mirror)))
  (pad "1" smd roundrect (at -1.4 0 90) (size 1.1 1.1) (layers "B.Cu" "B.Mask" "B.Paste") (roundrect_rratio 0.2272727273) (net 2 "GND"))
  (pad "2" smd roundrect (at 1.4 0 90) (size 1.1 1.1) (layers "B.Cu" "B.Mask" "B.Paste") (roundrect_rratio 0.2272727273) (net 3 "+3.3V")))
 (gr_arc (start 113 62) (mid 113.87868 59.87868) (end 116 59) (stroke (width 0.05) (type default)) (locked yes) (layer "Edge.Cuts"))
 (gr_arc (start 125 59) (mid 127.12132 59.87868) (end 128 62) (stroke (width 0.05) (type default)) (locked yes) (layer "Edge.Cuts"))
 (gr_line (start 125 79) (end 116 79) (stroke (width 0.05) (type default)) (locked yes) (layer "Edge.Cuts"))
 (gr_arc (start 128 76) (mid 127.12132 78.12132) (end 125 79) (stroke (width 0.05) (type default)) (locked yes) (layer "Edge.Cuts"))
 (gr_line (start 116 59) (end 125 59) (stroke (width 0.05) (type default)) (locked yes) (layer "Edge.Cuts"))
 (gr_arc (start 116 79) (mid 113.87868 78.12132) (end 113 76) (stroke (width 0.05) (type default)) (locked yes) (layer "Edge.Cuts"))
 (gr_line (start 128 62) (end 128 76) (stroke (width 0.05) (type default)) (locked yes) (layer "Edge.Cuts"))
 (gr_line (start 113 76) (end 113 62) (stroke (width 0.05) (type default)) (locked yes) (layer "Edge.Cuts"))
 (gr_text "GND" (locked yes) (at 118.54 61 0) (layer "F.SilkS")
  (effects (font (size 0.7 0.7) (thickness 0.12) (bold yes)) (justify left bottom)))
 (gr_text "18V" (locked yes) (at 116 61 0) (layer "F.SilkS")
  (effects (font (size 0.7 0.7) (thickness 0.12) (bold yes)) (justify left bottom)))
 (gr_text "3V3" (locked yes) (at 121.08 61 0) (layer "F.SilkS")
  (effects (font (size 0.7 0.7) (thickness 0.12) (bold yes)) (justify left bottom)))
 (segment (start 115.525 66) (end 115.525 63.895) (width 1.5) (locked yes) (layer "F.Cu") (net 1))
 (segment (start 115.525 69) (end 115.525 74.6351) (width 1.5) (locked yes) (layer "F.Cu") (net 1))
 (segment (start 115.525 74.6351) (end 117.1899 76.3) (width 1.5) (locked yes) (layer "F.Cu") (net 1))
 (segment (start 117.1899 76.3) (end 117.85 76.3) (width 1.5) (locked yes) (layer "F.Cu") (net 1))
 (segment (start 115.525 69) (end 115.525 66) (width 1.5) (locked yes) (layer "F.Cu") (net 1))
 (segment (start 115.525 63.895) (end 116.92 62.5) (width 1.5) (locked yes) (layer "F.Cu") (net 1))
 (segment (start 116.92 62.5) (end 116.92 65.92) (width 1.5) (locked yes) (layer "B.Cu") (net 1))
 (segment (start 116.92 65.92) (end 117 66) (width 1.5) (locked yes) (layer "B.Cu") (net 1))
 (segment (start 118.475 71.325) (end 118.85 71.7) (width 1.5) (locked yes) (layer "F.Cu") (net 2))
 (segment (start 121.525 69) (end 121.525 66) (width 1.5) (locked yes) (layer "F.Cu") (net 2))
 (segment (start 118.475 69) (end 118.475 71.325) (width 1.5) (locked yes) (layer "F.Cu") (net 2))
 (segment (start 118.475 69) (end 118.475 66) (width 1.5) (locked yes) (layer "F.Cu") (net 2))
 (segment (start 118.475 63.485) (end 119.46 62.5) (width 1.5) (locked yes) (layer "F.Cu") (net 2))
 (segment (start 118.475 66) (end 118.475 63.485) (width 1.5) (locked yes) (layer "F.Cu") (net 2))
 (segment (start 121.525 69) (end 118.475 69) (width 1.5) (locked yes) (layer "F.Cu") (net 2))
 (segment (start 119.46 63.935) (end 121.525 66) (width 1.5) (locked yes) (layer "F.Cu") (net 2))
 (segment (start 119.46 62.5) (end 119.46 63.935) (width 1.5) (locked yes) (layer "F.Cu") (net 2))
 (segment (start 119.46 62.5) (end 119.46 67.54) (width 1.5) (locked yes) (layer "B.Cu") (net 2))
 (segment (start 122 68.4) (end 120.32 68.4) (width 1.5) (locked yes) (layer "B.Cu") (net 2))
 (segment (start 120.32 68.4) (end 119.46 67.54) (width 1.5) (locked yes) (layer "B.Cu") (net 2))
 (segment (start 119.46 67.54) (end 117 70) (width 1.5) (locked yes) (layer "B.Cu") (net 2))
 (segment (start 124.475 69) (end 124.475 73.675) (width 1.5) (locked yes) (layer "F.Cu") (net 3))
 (segment (start 124.475 66) (end 124.475 64.975) (width 1.5) (locked yes) (layer "F.Cu") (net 3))
 (segment (start 124.475 69) (end 124.475 66) (width 1.5) (locked yes) (layer "F.Cu") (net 3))
 (segment (start 124.475 73.675) (end 124.15 74) (width 1.5) (locked yes) (layer "F.Cu") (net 3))
 (segment (start 117.85 74) (end 124.15 74) (width 1.5) (locked yes) (layer "F.Cu") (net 3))
 (segment (start 124.475 64.975) (end 122 62.5) (width 1.5) (locked yes) (layer "F.Cu") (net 3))
 (segment (start 122 62.5) (end 122 65.6) (width 1.5) (locked yes) (layer "B.Cu") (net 3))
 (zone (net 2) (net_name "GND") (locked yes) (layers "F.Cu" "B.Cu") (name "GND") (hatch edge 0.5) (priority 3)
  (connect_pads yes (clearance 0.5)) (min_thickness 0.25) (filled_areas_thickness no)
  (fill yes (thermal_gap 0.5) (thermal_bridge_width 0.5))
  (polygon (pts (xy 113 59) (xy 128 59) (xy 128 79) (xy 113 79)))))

